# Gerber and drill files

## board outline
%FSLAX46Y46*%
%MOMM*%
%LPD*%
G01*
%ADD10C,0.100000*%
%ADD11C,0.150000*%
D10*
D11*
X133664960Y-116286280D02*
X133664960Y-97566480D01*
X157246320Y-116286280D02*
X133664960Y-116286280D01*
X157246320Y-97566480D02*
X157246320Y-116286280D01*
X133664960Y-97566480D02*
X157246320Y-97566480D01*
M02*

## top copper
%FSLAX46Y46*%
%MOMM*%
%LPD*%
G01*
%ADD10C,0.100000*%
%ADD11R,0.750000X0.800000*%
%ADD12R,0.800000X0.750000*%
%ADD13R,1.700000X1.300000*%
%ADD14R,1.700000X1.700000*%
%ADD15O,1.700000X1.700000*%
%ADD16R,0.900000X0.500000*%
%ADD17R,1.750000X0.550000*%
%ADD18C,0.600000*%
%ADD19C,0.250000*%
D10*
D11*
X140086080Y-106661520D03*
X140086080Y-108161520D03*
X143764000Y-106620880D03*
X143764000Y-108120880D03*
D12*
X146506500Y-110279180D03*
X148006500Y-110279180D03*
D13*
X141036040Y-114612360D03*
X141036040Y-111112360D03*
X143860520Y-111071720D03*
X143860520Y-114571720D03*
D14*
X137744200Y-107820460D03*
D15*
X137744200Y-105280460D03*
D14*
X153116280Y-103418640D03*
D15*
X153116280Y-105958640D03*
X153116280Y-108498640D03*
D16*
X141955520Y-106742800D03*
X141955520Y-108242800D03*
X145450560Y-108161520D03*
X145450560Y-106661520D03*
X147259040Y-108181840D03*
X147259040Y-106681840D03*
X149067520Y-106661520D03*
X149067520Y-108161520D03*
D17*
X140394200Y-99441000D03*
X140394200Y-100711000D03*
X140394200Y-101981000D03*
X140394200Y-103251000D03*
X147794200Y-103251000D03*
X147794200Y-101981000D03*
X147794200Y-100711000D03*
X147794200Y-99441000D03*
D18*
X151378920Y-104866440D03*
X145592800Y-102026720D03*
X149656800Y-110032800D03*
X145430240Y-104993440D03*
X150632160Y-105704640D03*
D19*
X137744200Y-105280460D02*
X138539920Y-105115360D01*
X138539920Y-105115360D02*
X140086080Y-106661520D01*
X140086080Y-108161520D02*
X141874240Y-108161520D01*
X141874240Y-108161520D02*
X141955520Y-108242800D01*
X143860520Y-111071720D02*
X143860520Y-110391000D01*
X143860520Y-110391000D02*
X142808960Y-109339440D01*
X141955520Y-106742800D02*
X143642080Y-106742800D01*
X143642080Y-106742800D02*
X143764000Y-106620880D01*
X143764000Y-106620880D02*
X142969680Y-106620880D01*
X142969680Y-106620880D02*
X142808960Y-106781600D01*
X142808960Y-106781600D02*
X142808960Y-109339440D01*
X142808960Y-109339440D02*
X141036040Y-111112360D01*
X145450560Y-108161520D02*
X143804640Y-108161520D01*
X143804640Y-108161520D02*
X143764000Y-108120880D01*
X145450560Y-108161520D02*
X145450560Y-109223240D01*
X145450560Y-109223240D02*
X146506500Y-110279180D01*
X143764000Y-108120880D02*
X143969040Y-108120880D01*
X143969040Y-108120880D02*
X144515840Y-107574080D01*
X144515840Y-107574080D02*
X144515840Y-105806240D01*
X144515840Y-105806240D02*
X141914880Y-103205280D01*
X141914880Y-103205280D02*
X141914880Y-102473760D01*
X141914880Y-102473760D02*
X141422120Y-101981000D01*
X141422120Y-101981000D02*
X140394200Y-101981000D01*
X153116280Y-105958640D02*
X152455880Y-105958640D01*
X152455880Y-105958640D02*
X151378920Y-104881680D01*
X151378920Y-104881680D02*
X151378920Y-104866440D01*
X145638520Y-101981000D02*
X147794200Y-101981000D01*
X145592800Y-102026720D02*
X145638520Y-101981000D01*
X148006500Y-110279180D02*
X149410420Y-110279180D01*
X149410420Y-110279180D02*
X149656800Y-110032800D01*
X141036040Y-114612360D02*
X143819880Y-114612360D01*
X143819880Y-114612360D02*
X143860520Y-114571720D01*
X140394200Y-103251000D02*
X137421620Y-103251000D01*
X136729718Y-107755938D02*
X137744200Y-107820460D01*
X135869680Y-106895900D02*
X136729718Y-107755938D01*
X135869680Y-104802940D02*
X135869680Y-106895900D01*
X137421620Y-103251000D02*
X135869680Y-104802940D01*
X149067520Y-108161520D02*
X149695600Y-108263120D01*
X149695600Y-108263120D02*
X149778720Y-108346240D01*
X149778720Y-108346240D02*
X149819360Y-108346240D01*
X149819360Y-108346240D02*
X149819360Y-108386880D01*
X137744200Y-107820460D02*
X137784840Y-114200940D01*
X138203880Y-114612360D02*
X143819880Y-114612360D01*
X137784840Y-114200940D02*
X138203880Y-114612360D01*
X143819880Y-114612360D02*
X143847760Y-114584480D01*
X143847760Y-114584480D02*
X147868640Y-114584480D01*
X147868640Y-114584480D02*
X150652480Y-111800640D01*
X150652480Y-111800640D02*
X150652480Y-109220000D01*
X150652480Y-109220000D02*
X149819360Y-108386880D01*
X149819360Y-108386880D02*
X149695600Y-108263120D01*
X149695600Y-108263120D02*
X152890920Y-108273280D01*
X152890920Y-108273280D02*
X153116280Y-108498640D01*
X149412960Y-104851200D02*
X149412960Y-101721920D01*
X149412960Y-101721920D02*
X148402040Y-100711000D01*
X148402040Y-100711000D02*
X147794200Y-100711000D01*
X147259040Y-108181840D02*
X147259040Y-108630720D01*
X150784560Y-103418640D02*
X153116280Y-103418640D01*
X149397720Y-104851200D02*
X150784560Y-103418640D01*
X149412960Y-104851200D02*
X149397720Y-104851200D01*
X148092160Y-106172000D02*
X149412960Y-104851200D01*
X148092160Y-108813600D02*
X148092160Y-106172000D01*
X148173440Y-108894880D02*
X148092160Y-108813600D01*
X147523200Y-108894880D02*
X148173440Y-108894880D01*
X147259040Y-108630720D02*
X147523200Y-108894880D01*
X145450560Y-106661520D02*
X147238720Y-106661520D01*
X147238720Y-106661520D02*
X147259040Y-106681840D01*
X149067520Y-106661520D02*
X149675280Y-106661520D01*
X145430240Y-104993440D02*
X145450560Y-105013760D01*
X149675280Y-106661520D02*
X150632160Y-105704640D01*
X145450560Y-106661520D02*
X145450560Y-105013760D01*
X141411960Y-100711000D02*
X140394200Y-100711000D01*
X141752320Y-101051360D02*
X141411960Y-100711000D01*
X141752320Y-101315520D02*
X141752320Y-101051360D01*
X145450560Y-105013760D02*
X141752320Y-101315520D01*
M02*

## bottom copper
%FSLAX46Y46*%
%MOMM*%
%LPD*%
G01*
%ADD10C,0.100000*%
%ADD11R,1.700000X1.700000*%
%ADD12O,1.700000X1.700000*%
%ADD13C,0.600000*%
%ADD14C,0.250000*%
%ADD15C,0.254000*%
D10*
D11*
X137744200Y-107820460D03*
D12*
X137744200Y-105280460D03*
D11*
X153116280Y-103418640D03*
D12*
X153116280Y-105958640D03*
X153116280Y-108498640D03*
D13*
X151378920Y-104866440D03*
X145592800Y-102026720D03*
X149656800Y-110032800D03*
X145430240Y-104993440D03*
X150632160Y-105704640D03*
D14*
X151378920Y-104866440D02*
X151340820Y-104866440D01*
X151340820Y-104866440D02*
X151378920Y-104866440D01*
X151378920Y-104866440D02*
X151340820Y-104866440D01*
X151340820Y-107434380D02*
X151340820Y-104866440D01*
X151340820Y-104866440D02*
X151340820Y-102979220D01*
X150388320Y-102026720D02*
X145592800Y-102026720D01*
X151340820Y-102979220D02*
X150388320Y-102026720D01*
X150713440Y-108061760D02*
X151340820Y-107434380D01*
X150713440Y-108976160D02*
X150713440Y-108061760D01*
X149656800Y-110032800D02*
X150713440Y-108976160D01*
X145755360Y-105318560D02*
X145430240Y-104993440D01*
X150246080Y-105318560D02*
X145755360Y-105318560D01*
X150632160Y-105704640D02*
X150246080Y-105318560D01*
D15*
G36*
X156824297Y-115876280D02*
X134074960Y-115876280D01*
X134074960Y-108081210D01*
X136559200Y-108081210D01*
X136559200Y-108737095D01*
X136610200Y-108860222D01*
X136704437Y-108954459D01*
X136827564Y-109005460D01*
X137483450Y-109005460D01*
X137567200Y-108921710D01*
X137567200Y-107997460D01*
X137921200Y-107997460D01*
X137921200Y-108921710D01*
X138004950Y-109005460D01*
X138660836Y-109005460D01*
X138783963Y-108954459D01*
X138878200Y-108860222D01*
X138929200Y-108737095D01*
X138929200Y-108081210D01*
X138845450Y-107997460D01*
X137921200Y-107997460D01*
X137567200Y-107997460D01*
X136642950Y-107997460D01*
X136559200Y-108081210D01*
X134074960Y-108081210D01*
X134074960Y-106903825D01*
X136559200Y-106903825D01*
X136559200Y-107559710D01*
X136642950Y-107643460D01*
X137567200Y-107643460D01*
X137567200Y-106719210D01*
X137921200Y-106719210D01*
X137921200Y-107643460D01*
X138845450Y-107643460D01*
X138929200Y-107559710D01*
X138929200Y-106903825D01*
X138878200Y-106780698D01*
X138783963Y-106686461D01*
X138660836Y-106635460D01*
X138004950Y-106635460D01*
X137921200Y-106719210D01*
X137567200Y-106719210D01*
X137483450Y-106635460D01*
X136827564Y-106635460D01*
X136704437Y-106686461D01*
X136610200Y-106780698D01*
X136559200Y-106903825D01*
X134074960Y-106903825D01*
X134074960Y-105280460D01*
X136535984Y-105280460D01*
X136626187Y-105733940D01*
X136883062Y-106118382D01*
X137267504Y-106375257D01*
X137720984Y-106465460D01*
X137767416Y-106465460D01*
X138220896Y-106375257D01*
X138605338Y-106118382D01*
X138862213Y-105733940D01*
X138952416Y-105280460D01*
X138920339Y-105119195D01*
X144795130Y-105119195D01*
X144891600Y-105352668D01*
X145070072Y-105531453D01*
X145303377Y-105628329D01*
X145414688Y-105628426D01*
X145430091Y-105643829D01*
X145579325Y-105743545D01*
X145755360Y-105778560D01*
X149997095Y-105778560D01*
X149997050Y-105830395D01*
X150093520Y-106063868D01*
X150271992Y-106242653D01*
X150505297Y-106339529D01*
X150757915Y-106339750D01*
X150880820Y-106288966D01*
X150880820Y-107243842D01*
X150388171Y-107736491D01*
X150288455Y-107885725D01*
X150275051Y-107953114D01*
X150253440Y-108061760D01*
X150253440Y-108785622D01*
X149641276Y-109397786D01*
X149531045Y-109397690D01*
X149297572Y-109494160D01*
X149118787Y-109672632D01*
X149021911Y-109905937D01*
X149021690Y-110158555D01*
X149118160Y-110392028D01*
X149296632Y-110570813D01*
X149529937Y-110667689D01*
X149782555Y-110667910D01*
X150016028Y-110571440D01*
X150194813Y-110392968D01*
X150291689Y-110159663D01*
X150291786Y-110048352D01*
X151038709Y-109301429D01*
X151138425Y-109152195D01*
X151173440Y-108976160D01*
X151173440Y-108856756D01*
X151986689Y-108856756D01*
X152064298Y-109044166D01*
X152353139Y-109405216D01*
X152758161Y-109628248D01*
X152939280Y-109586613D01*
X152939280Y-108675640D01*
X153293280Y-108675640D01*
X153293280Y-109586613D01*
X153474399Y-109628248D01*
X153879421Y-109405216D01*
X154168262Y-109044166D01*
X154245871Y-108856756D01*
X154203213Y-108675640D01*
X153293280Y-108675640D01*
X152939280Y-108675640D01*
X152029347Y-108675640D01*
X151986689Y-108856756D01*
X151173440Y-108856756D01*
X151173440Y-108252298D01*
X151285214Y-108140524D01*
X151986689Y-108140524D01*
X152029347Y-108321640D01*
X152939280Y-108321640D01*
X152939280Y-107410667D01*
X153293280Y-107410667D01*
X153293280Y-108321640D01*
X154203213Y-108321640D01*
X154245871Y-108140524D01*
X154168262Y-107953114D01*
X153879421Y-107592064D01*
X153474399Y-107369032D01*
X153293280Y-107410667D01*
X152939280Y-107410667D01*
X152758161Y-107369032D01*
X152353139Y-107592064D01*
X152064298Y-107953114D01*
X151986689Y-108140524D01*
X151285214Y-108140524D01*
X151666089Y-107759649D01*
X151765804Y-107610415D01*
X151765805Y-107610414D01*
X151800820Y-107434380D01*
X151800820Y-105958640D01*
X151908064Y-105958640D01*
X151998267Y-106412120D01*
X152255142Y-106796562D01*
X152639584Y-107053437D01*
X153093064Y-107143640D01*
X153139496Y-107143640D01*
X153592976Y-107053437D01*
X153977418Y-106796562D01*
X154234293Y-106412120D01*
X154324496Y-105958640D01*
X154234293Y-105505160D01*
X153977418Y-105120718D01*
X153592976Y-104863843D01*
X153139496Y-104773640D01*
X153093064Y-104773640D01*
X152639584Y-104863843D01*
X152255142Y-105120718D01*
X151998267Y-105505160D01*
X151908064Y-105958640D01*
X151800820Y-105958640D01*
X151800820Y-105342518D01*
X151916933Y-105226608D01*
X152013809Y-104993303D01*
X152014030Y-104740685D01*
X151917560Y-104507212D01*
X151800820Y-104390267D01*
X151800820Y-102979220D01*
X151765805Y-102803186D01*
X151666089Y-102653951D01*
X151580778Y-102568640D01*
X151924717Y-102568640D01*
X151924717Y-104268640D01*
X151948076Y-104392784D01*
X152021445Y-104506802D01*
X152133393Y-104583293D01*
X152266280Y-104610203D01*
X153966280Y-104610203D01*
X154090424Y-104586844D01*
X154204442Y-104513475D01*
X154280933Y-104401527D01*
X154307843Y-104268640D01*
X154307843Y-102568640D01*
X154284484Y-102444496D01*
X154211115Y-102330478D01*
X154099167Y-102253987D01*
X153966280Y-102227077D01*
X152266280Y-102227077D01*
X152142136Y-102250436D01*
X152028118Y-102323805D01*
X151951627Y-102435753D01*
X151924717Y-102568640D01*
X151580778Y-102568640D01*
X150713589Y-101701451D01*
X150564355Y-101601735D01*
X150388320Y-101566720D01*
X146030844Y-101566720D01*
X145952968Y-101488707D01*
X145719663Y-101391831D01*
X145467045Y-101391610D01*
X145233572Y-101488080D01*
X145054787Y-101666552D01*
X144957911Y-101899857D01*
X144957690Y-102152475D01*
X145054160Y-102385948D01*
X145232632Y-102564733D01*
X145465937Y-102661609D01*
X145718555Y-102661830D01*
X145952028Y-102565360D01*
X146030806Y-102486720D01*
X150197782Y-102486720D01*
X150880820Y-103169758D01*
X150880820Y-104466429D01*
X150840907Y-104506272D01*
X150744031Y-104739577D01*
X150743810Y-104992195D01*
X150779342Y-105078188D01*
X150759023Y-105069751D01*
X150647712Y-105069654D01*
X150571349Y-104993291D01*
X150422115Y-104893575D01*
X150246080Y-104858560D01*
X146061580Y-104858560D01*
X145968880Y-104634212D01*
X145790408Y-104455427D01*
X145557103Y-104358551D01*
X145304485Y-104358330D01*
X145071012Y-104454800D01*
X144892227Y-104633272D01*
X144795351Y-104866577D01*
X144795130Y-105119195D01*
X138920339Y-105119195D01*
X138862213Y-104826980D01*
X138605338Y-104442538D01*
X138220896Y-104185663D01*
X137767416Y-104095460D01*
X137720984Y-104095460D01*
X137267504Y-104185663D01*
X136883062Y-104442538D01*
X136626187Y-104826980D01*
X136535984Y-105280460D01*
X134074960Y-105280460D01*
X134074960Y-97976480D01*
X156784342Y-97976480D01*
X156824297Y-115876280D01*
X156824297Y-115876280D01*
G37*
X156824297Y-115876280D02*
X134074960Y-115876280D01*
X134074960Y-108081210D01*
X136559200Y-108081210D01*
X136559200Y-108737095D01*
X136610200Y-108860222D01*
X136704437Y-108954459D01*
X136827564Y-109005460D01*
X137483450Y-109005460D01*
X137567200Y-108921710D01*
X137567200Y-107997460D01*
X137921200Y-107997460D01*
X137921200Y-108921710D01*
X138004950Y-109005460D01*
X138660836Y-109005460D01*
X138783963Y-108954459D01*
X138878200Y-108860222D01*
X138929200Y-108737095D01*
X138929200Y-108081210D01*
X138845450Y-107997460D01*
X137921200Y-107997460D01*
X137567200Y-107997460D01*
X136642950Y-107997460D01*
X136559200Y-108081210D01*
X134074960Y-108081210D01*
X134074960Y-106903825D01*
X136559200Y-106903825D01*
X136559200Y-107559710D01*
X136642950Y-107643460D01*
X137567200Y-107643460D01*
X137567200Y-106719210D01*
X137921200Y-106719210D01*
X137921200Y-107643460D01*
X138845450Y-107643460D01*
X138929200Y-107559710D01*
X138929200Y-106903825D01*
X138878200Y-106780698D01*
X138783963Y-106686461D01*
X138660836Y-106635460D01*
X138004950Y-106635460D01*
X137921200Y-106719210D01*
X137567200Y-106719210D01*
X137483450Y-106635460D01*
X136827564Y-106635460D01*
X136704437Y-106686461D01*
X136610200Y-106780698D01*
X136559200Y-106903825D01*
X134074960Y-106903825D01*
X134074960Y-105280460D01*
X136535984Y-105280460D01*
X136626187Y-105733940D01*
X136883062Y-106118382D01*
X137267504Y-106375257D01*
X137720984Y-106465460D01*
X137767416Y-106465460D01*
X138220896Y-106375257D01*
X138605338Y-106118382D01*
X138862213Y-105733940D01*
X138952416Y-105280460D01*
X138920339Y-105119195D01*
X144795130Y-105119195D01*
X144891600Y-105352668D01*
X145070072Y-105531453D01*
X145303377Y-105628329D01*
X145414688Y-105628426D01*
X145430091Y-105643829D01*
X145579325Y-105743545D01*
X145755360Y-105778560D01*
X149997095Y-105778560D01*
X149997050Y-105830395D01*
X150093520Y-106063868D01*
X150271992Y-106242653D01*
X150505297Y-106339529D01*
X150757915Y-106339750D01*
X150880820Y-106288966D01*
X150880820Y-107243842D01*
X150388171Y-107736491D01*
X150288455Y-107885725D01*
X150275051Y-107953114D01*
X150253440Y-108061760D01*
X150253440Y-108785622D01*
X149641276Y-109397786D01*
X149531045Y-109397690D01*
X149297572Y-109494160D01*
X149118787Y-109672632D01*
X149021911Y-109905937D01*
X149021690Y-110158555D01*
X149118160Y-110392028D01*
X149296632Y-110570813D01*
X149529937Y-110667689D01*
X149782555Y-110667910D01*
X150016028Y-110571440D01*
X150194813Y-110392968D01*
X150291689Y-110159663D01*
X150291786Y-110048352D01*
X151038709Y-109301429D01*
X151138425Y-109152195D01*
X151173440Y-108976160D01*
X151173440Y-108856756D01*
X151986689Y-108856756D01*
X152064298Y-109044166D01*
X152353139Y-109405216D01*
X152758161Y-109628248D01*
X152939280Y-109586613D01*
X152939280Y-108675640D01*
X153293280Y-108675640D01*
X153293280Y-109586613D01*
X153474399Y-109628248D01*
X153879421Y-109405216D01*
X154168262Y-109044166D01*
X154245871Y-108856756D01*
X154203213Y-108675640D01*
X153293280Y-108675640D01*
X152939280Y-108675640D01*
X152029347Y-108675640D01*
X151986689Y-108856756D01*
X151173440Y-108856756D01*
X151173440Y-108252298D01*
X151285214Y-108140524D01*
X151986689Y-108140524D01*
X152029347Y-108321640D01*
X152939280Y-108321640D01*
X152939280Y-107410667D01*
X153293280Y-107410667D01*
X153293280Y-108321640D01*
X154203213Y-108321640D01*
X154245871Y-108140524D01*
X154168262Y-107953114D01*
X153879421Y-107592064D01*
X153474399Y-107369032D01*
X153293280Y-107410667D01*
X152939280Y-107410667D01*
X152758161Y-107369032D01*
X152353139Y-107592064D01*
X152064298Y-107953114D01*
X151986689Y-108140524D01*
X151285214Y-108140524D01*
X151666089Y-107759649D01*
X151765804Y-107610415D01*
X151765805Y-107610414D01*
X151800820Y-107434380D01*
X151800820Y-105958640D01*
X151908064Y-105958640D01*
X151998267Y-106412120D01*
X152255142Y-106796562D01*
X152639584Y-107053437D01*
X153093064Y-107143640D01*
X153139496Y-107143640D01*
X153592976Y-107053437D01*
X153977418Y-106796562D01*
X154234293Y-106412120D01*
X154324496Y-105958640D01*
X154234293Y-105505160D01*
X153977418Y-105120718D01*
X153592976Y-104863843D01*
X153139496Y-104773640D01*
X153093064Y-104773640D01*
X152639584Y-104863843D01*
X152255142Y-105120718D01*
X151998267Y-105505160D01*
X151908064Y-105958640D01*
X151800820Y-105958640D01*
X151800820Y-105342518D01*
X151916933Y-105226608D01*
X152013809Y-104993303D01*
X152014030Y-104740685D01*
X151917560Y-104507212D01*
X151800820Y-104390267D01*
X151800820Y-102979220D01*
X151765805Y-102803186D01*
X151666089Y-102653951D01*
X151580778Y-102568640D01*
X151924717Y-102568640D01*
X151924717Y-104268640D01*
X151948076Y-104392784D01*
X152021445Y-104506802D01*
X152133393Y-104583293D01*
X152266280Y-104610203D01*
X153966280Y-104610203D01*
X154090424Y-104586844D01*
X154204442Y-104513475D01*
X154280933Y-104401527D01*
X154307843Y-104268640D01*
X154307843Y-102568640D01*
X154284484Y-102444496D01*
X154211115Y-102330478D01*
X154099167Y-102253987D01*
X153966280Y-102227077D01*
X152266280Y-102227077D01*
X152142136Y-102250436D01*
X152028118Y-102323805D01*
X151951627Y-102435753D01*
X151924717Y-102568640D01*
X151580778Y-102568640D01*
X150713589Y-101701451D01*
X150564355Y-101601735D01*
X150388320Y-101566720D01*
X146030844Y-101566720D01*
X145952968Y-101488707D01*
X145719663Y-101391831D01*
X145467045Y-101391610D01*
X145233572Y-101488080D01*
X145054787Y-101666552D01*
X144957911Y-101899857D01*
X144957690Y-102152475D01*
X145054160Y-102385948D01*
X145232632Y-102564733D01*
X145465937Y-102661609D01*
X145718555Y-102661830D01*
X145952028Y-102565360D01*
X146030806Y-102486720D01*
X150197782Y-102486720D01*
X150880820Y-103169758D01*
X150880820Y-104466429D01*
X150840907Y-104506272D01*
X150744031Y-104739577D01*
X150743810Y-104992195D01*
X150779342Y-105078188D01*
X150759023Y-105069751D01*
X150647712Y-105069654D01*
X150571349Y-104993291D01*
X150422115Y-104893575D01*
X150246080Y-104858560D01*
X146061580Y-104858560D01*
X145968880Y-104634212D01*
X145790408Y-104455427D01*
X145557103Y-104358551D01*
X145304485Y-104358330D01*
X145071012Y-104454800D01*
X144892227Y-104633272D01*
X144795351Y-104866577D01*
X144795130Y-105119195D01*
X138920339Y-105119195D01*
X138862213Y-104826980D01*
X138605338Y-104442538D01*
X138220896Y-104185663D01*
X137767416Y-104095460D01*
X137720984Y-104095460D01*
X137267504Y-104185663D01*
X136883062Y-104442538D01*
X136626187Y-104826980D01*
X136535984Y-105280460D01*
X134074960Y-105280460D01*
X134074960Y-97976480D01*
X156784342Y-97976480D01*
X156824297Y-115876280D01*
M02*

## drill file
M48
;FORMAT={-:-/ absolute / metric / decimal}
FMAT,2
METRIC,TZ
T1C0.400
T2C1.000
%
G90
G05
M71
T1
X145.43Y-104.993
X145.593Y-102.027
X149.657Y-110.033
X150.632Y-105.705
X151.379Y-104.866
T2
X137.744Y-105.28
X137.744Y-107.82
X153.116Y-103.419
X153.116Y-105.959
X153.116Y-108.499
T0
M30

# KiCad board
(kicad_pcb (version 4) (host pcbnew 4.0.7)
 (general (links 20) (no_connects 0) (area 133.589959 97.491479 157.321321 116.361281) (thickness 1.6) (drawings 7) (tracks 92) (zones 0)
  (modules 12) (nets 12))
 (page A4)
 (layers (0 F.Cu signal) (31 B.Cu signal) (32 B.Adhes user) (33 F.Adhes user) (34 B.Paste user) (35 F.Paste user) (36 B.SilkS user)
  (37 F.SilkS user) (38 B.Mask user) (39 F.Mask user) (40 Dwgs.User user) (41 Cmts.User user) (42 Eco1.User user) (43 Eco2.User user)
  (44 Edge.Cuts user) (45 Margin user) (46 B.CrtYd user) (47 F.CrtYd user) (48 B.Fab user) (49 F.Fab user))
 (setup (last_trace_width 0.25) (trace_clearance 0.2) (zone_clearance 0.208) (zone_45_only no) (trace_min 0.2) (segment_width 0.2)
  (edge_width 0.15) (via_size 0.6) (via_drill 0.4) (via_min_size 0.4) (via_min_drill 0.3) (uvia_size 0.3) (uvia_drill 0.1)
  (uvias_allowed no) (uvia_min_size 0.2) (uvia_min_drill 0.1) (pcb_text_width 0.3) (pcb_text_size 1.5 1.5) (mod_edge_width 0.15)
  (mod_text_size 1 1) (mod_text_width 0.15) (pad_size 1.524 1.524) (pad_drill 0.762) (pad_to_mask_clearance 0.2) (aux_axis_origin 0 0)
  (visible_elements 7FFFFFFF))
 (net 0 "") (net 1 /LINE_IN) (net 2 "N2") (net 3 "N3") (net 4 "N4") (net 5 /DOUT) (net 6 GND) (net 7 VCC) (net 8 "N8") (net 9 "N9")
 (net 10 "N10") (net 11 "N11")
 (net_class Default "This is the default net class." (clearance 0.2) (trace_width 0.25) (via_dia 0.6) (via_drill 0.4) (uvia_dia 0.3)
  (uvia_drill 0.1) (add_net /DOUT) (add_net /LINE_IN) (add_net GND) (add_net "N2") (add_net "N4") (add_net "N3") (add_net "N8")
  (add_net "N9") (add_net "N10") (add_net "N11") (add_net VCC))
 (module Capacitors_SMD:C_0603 (layer F.Cu) (at 140.08608 107.41152 90)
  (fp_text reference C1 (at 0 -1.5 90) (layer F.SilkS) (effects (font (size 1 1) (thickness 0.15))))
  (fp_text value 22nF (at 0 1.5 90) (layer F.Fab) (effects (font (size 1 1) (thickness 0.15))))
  (pad 2 smd rect (at 0.75 0 90) (size 0.8 0.75) (layers F.Cu F.Paste F.Mask) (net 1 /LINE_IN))
  (pad 1 smd rect (at -0.75 0 90) (size 0.8 0.75) (layers F.Cu F.Paste F.Mask) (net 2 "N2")))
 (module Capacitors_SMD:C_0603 (layer F.Cu) (at 143.764 107.37088 90)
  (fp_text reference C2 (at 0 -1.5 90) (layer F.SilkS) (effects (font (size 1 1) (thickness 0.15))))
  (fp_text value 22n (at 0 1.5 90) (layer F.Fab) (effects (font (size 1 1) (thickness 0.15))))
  (pad 2 smd rect (at 0.75 0 90) (size 0.8 0.75) (layers F.Cu F.Paste F.Mask) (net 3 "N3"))
  (pad 1 smd rect (at -0.75 0 90) (size 0.8 0.75) (layers F.Cu F.Paste F.Mask) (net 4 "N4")))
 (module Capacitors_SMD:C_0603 (layer F.Cu) (at 147.2565 110.27918 180)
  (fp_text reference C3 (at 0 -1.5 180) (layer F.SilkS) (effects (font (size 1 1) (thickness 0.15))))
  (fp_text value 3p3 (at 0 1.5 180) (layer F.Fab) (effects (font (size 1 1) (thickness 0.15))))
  (pad 2 smd rect (at 0.75 0 180) (size 0.8 0.75) (layers F.Cu F.Paste F.Mask) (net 4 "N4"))
  (pad 1 smd rect (at -0.75 0 180) (size 0.8 0.75) (layers F.Cu F.Paste F.Mask) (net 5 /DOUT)))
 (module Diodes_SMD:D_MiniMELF (layer F.Cu) (at 141.03604 112.86236 90)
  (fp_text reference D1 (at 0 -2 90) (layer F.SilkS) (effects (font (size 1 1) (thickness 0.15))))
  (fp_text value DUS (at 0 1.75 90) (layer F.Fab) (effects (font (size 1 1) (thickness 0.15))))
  (pad 1 smd rect (at -1.75 0 90) (size 1.3 1.7) (layers F.Cu F.Paste F.Mask) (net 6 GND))
  (pad 2 smd rect (at 1.75 0 90) (size 1.3 1.7) (layers F.Cu F.Paste F.Mask) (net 3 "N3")))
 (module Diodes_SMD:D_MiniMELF (layer F.Cu) (at 143.86052 112.82172 270)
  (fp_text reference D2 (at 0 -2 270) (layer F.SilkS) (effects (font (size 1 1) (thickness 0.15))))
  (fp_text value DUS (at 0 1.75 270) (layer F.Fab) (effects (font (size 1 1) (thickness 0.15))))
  (pad 1 smd rect (at -1.75 0 270) (size 1.3 1.7) (layers F.Cu F.Paste F.Mask) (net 3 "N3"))
  (pad 2 smd rect (at 1.75 0 270) (size 1.3 1.7) (layers F.Cu F.Paste F.Mask) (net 6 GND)))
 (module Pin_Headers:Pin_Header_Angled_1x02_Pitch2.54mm (layer F.Cu) (at 137.7442 107.82046 180)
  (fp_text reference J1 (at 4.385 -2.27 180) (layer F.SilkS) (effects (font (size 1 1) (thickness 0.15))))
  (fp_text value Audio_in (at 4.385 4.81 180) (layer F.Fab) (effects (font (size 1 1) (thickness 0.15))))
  (pad 1 thru_hole rect (at 0 0 180) (size 1.7 1.7) (drill 1) (layers *.Cu *.Mask) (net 6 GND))
  (pad 2 thru_hole oval (at 0 2.54 180) (size 1.7 1.7) (drill 1) (layers *.Cu *.Mask) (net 1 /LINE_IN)))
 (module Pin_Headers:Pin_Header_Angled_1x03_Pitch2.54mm (layer F.Cu) (at 153.11628 103.41864)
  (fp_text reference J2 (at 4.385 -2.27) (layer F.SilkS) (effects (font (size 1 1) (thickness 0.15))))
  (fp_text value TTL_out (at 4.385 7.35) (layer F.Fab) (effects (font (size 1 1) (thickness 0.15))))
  (pad 1 thru_hole rect (at 0 0) (size 1.7 1.7) (drill 1) (layers *.Cu *.Mask) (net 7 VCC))
  (pad 2 thru_hole oval (at 0 2.54) (size 1.7 1.7) (drill 1) (layers *.Cu *.Mask) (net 5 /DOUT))
  (pad 3 thru_hole oval (at 0 5.08) (size 1.7 1.7) (drill 1) (layers *.Cu *.Mask) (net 6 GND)))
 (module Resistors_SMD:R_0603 (layer F.Cu) (at 141.95552 107.4928 270)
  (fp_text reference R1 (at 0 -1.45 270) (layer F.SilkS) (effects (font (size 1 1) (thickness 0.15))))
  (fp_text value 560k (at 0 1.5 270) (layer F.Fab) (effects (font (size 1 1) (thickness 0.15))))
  (pad 1 smd rect (at -0.75 0 270) (size 0.5 0.9) (layers F.Cu F.Paste F.Mask) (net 3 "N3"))
  (pad 2 smd rect (at 0.75 0 270) (size 0.5 0.9) (layers F.Cu F.Paste F.Mask) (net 2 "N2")))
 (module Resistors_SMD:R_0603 (layer F.Cu) (at 145.45056 107.41152 90)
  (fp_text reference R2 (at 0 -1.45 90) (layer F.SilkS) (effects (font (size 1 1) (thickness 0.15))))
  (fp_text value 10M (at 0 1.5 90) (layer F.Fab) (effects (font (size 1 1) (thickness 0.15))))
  (pad 1 smd rect (at -0.75 0 90) (size 0.5 0.9) (layers F.Cu F.Paste F.Mask) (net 4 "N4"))
  (pad 2 smd rect (at 0.75 0 90) (size 0.5 0.9) (layers F.Cu F.Paste F.Mask) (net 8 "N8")))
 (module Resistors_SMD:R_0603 (layer F.Cu) (at 147.25904 107.43184 90)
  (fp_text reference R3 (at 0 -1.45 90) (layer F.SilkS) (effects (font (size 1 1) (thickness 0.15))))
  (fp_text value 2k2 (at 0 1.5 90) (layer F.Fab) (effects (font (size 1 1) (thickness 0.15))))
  (pad 1 smd rect (at -0.75 0 90) (size 0.5 0.9) (layers F.Cu F.Paste F.Mask) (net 7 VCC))
  (pad 2 smd rect (at 0.75 0 90) (size 0.5 0.9) (layers F.Cu F.Paste F.Mask) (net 8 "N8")))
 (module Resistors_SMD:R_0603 (layer F.Cu) (at 149.06752 107.41152 270)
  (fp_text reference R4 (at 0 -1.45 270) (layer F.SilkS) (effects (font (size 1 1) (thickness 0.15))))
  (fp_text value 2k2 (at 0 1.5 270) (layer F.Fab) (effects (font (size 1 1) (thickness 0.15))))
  (pad 1 smd rect (at -0.75 0 270) (size 0.5 0.9) (layers F.Cu F.Paste F.Mask) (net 8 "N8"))
  (pad 2 smd rect (at 0.75 0 270) (size 0.5 0.9) (layers F.Cu F.Paste F.Mask) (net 6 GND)))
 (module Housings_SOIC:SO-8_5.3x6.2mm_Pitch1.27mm (layer F.Cu) (at 144.0942 101.346)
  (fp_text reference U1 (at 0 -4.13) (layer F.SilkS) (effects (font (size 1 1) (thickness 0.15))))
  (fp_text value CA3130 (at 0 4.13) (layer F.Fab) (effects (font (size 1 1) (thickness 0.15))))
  (pad 1 smd rect (at -3.7 -1.905) (size 1.75 0.55) (layers F.Cu F.Paste F.Mask) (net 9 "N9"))
  (pad 2 smd rect (at -3.7 -0.635) (size 1.75 0.55) (layers F.Cu F.Paste F.Mask) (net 8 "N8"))
  (pad 3 smd rect (at -3.7 0.635) (size 1.75 0.55) (layers F.Cu F.Paste F.Mask) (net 4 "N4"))
  (pad 4 smd rect (at -3.7 1.905) (size 1.75 0.55) (layers F.Cu F.Paste F.Mask) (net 6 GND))
  (pad 5 smd rect (at 3.7 1.905) (size 1.75 0.55) (layers F.Cu F.Paste F.Mask) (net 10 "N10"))
  (pad 6 smd rect (at 3.7 0.635) (size 1.75 0.55) (layers F.Cu F.Paste F.Mask) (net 5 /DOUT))
  (pad 7 smd rect (at 3.7 -0.635) (size 1.75 0.55) (layers F.Cu F.Paste F.Mask) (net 7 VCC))
  (pad 8 smd rect (at 3.7 -1.905) (size 1.75 0.55) (layers F.Cu F.Paste F.Mask) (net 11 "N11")))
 (gr_line (start 133.66496 116.28628) (end 133.66496 97.56648) (angle 90) (layer Edge.Cuts) (width 0.15))
 (gr_line (start 157.24632 116.28628) (end 133.66496 116.28628) (angle 90) (layer Edge.Cuts) (width 0.15))
 (gr_line (start 157.24632 97.56648) (end 157.24632 116.28628) (angle 90) (layer Edge.Cuts) (width 0.15))
 (gr_line (start 133.66496 97.56648) (end 157.24632 97.56648) (angle 90) (layer Edge.Cuts) (width 0.15))
 (segment (start 137.7442 105.28046) (end 138.53992 105.11536) (width 0.25) (layer F.Cu) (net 1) (status 10))
 (segment (start 138.53992 105.11536) (end 140.08608 106.66152) (width 0.25) (layer F.Cu) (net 1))
 (segment (start 140.08608 108.16152) (end 141.87424 108.16152) (width 0.25) (layer F.Cu) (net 2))
 (segment (start 141.87424 108.16152) (end 141.95552 108.2428) (width 0.25) (layer F.Cu) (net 2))
 (segment (start 143.86052 111.07172) (end 143.86052 110.391) (width 0.25) (layer F.Cu) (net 3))
 (segment (start 143.86052 110.391) (end 142.80896 109.33944) (width 0.25) (layer F.Cu) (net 3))
 (segment (start 141.95552 106.7428) (end 143.64208 106.7428) (width 0.25) (layer F.Cu) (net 3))
 (segment (start 143.64208 106.7428) (end 143.764 106.62088) (width 0.25) (layer F.Cu) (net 3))
 (segment (start 143.764 106.62088) (end 142.96968 106.62088) (width 0.25) (layer F.Cu) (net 3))
 (segment (start 142.96968 106.62088) (end 142.80896 106.7816) (width 0.25) (layer F.Cu) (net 3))
 (segment (start 142.80896 106.7816) (end 142.80896 109.33944) (width 0.25) (layer F.Cu) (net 3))
 (segment (start 142.80896 109.33944) (end 141.03604 111.11236) (width 0.25) (layer F.Cu) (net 3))
 (segment (start 145.45056 108.16152) (end 143.80464 108.16152) (width 0.25) (layer F.Cu) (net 4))
 (segment (start 143.80464 108.16152) (end 143.764 108.12088) (width 0.25) (layer F.Cu) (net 4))
 (segment (start 145.45056 108.16152) (end 145.45056 109.22324) (width 0.25) (layer F.Cu) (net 4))
 (segment (start 145.45056 109.22324) (end 146.5065 110.27918) (width 0.25) (layer F.Cu) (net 4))
 (segment (start 143.764 108.12088) (end 143.96904 108.12088) (width 0.25) (layer F.Cu) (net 4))
 (segment (start 143.96904 108.12088) (end 144.51584 107.57408) (width 0.25) (layer F.Cu) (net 4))
 (segment (start 144.51584 107.57408) (end 144.51584 105.80624) (width 0.25) (layer F.Cu) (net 4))
 (segment (start 144.51584 105.80624) (end 141.91488 103.20528) (width 0.25) (layer F.Cu) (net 4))
 (segment (start 141.91488 103.20528) (end 141.91488 102.47376) (width 0.25) (layer F.Cu) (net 4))
 (segment (start 141.91488 102.47376) (end 141.42212 101.981) (width 0.25) (layer F.Cu) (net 4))
 (segment (start 141.42212 101.981) (end 140.3942 101.981) (width 0.25) (layer F.Cu) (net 4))
 (segment (start 153.11628 105.95864) (end 152.45588 105.95864) (width 0.25) (layer F.Cu) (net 5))
 (segment (start 152.45588 105.95864) (end 151.37892 104.88168) (width 0.25) (layer F.Cu) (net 5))
 (segment (start 151.37892 104.88168) (end 151.37892 104.86644) (width 0.25) (layer F.Cu) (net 5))
 (via (at 151.37892 104.86644) (size 0.6) (drill 0.4) (layers F.Cu B.Cu) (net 5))
 (segment (start 151.37892 104.86644) (end 151.34082 104.86644) (width 0.25) (layer B.Cu) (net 5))
 (segment (start 151.34082 104.86644) (end 151.37892 104.86644) (width 0.25) (layer B.Cu) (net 5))
 (segment (start 151.37892 104.86644) (end 151.34082 104.86644) (width 0.25) (layer B.Cu) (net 5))
 (segment (start 151.34082 107.43438) (end 151.34082 104.86644) (width 0.25) (layer B.Cu) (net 5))
 (segment (start 151.34082 104.86644) (end 151.34082 102.97922) (width 0.25) (layer B.Cu) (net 5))
 (segment (start 145.63852 101.981) (end 147.7942 101.981) (width 0.25) (layer F.Cu) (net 5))
 (segment (start 145.5928 102.02672) (end 145.63852 101.981) (width 0.25) (layer F.Cu) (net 5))
 (via (at 145.5928 102.02672) (size 0.6) (drill 0.4) (layers F.Cu B.Cu) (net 5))
 (segment (start 150.38832 102.02672) (end 145.5928 102.02672) (width 0.25) (layer B.Cu) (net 5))
 (segment (start 151.34082 102.97922) (end 150.38832 102.02672) (width 0.25) (layer B.Cu) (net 5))
 (segment (start 148.0065 110.27918) (end 149.41042 110.27918) (width 0.25) (layer F.Cu) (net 5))
 (segment (start 150.71344 108.06176) (end 151.34082 107.43438) (width 0.25) (layer B.Cu) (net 5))
 (segment (start 150.71344 108.97616) (end 150.71344 108.06176) (width 0.25) (layer B.Cu) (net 5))
 (segment (start 149.6568 110.0328) (end 150.71344 108.97616) (width 0.25) (layer B.Cu) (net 5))
 (via (at 149.6568 110.0328) (size 0.6) (drill 0.4) (layers F.Cu B.Cu) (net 5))
 (segment (start 149.41042 110.27918) (end 149.6568 110.0328) (width 0.25) (layer F.Cu) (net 5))
 (segment (start 141.03604 114.61236) (end 143.81988 114.61236) (width 0.25) (layer F.Cu) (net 6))
 (segment (start 143.81988 114.61236) (end 143.86052 114.57172) (width 0.25) (layer F.Cu) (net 6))
 (segment (start 140.3942 103.251) (end 137.42162 103.251) (width 0.25) (layer F.Cu) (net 6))
 (segment (start 136.729718 107.755938) (end 137.7442 107.82046) (width 0.25) (layer F.Cu) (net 6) (status 20))
 (segment (start 135.86968 106.8959) (end 136.729718 107.755938) (width 0.25) (layer F.Cu) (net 6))
 (segment (start 135.86968 104.80294) (end 135.86968 106.8959) (width 0.25) (layer F.Cu) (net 6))
 (segment (start 137.42162 103.251) (end 135.86968 104.80294) (width 0.25) (layer F.Cu) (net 6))
 (segment (start 149.06752 108.16152) (end 149.6956 108.26312) (width 0.25) (layer F.Cu) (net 6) (status 10))
 (segment (start 149.6956 108.26312) (end 149.77872 108.34624) (width 0.25) (layer F.Cu) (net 6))
 (segment (start 149.77872 108.34624) (end 149.81936 108.34624) (width 0.25) (layer F.Cu) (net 6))
 (segment (start 149.81936 108.34624) (end 149.81936 108.38688) (width 0.25) (layer F.Cu) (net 6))
 (segment (start 137.7442 107.82046) (end 137.78484 114.20094) (width 0.25) (layer F.Cu) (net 6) (status 10))
 (segment (start 138.20388 114.61236) (end 143.81988 114.61236) (width 0.25) (layer F.Cu) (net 6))
 (segment (start 137.78484 114.20094) (end 138.20388 114.61236) (width 0.25) (layer F.Cu) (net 6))
 (segment (start 143.81988 114.61236) (end 143.84776 114.58448) (width 0.25) (layer F.Cu) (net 6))
 (segment (start 143.84776 114.58448) (end 147.86864 114.58448) (width 0.25) (layer F.Cu) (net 6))
 (segment (start 147.86864 114.58448) (end 150.65248 111.80064) (width 0.25) (layer F.Cu) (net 6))
 (segment (start 150.65248 111.80064) (end 150.65248 109.22) (width 0.25) (layer F.Cu) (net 6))
 (segment (start 150.65248 109.22) (end 149.81936 108.38688) (width 0.25) (layer F.Cu) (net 6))
 (segment (start 149.81936 108.38688) (end 149.6956 108.26312) (width 0.25) (layer F.Cu) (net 6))
 (segment (start 149.6956 108.26312) (end 152.89092 108.27328) (width 0.25) (layer F.Cu) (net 6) (status 20))
 (segment (start 152.89092 108.27328) (end 153.11628 108.49864) (width 0.25) (layer F.Cu) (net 6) (status 30))
 (segment (start 149.41296 104.8512) (end 149.41296 101.72192) (width 0.25) (layer F.Cu) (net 7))
 (segment (start 149.41296 101.72192) (end 148.40204 100.711) (width 0.25) (layer F.Cu) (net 7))
 (segment (start 148.40204 100.711) (end 147.7942 100.711) (width 0.25) (layer F.Cu) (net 7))
 (segment (start 147.25904 108.18184) (end 147.25904 108.63072) (width 0.25) (layer F.Cu) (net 7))
 (segment (start 150.78456 103.41864) (end 153.11628 103.41864) (width 0.25) (layer F.Cu) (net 7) (status 20))
 (segment (start 149.39772 104.8512) (end 150.78456 103.41864) (width 0.25) (layer F.Cu) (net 7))
 (segment (start 149.41296 104.8512) (end 149.39772 104.8512) (width 0.25) (layer F.Cu) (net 7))
 (segment (start 148.09216 106.172) (end 149.41296 104.8512) (width 0.25) (layer F.Cu) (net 7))
 (segment (start 148.09216 108.8136) (end 148.09216 106.172) (width 0.25) (layer F.Cu) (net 7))
 (segment (start 148.17344 108.89488) (end 148.09216 108.8136) (width 0.25) (layer F.Cu) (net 7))
 (segment (start 147.5232 108.89488) (end 148.17344 108.89488) (width 0.25) (layer F.Cu) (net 7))
 (segment (start 147.25904 108.63072) (end 147.5232 108.89488) (width 0.25) (layer F.Cu) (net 7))
 (segment (start 145.45056 106.66152) (end 147.23872 106.66152) (width 0.25) (layer F.Cu) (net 8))
 (segment (start 147.23872 106.66152) (end 147.25904 106.68184) (width 0.25) (layer F.Cu) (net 8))
 (segment (start 149.06752 106.66152) (end 149.67528 106.66152) (width 0.25) (layer F.Cu) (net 8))
 (segment (start 145.43024 104.99344) (end 145.45056 105.01376) (width 0.25) (layer F.Cu) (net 8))
 (via (at 145.43024 104.99344) (size 0.6) (drill 0.4) (layers F.Cu B.Cu) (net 8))
 (segment (start 145.75536 105.31856) (end 145.43024 104.99344) (width 0.25) (layer B.Cu) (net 8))
 (segment (start 150.24608 105.31856) (end 145.75536 105.31856) (width 0.25) (layer B.Cu) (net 8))
 (segment (start 150.63216 105.70464) (end 150.24608 105.31856) (width 0.25) (layer B.Cu) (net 8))
 (via (at 150.63216 105.70464) (size 0.6) (drill 0.4) (layers F.Cu B.Cu) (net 8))
 (segment (start 149.67528 106.66152) (end 150.63216 105.70464) (width 0.25) (layer F.Cu) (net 8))
 (segment (start 145.45056 106.66152) (end 145.45056 105.01376) (width 0.25) (layer F.Cu) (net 8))
 (segment (start 141.41196 100.711) (end 140.3942 100.711) (width 0.25) (layer F.Cu) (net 8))
 (segment (start 141.75232 101.05136) (end 141.41196 100.711) (width 0.25) (layer F.Cu) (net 8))
 (segment (start 141.75232 101.31552) (end 141.75232 101.05136) (width 0.25) (layer F.Cu) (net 8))
 (segment (start 145.45056 105.01376) (end 141.75232 101.31552) (width 0.25) (layer F.Cu) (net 8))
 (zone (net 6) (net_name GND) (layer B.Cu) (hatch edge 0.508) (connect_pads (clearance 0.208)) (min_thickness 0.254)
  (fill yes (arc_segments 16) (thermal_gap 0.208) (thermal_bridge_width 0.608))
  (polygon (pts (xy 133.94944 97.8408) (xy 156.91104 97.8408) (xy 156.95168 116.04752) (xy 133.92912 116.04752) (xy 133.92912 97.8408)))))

